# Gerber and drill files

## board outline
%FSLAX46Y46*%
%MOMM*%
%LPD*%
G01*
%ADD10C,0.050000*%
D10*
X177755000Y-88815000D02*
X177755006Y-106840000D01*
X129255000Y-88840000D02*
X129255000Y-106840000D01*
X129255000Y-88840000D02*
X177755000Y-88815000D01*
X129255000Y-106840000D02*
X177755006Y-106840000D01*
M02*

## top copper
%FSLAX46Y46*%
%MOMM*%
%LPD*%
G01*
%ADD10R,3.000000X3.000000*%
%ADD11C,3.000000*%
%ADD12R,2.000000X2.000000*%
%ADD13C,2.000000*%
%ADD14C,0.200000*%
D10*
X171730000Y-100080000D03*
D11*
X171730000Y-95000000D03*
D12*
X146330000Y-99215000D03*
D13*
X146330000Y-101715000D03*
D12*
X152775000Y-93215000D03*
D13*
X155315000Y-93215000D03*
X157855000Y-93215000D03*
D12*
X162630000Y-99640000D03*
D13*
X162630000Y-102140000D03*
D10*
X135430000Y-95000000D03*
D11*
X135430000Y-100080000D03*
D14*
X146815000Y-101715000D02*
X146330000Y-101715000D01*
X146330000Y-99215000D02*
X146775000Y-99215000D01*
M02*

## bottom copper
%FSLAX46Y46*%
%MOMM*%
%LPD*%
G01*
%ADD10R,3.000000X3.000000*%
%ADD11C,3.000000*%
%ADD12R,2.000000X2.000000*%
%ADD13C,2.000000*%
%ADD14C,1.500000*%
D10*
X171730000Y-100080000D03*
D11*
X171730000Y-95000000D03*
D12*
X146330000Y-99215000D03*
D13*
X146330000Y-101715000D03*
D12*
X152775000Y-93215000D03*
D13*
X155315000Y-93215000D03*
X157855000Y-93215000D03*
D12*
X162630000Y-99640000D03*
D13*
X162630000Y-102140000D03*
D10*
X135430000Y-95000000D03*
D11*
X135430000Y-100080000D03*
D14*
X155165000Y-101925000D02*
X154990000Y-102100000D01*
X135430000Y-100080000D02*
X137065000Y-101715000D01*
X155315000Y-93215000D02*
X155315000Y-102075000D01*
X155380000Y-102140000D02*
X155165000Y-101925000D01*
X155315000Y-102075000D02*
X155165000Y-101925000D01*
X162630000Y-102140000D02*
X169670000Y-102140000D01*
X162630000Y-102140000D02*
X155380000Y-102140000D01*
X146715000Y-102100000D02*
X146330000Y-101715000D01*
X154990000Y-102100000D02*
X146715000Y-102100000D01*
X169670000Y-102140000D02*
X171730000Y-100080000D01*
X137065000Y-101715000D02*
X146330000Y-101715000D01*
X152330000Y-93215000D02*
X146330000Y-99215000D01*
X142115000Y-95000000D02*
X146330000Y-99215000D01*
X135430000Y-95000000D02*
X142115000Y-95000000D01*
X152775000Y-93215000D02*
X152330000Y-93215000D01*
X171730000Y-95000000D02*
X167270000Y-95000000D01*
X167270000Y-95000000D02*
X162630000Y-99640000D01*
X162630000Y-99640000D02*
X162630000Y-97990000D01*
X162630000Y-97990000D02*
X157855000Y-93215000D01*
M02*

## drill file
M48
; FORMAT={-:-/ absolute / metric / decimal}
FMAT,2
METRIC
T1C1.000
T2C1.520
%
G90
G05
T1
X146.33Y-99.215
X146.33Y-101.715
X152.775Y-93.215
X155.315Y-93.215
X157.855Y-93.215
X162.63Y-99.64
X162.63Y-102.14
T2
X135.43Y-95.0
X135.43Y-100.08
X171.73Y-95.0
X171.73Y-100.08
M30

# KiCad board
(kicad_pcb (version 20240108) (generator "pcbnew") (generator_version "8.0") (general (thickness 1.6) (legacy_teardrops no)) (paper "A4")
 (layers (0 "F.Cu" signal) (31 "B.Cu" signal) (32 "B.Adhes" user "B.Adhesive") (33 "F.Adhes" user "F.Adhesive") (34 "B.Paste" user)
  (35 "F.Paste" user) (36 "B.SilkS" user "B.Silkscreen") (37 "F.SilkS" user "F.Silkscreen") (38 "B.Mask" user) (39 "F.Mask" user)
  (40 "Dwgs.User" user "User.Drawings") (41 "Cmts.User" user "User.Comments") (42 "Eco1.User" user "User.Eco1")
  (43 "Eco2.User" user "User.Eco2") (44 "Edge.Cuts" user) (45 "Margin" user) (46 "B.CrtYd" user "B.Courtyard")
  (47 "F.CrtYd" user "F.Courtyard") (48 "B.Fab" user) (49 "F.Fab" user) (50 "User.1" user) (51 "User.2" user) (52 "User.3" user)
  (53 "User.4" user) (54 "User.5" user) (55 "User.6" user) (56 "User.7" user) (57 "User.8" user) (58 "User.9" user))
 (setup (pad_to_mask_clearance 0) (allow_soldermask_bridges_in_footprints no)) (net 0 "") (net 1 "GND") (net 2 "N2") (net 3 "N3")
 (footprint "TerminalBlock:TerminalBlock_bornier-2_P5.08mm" (layer "F.Cu") (at 171.73 100.08 90)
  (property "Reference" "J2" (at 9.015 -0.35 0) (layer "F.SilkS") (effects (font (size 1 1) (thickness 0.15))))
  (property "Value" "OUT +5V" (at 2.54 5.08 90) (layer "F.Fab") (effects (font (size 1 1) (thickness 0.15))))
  (pad "1" thru_hole rect (at 0 0 90) (size 3 3) (drill 1.52) (layers "*.Cu" "*.Mask") (remove_unused_layers no) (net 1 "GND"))
  (pad "2" thru_hole circle (at 5.08 0 90) (size 3 3) (drill 1.52) (layers "*.Cu" "*.Mask") (remove_unused_layers no) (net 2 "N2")))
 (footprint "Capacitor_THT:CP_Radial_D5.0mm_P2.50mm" (layer "F.Cu") (at 146.33 99.215 -90)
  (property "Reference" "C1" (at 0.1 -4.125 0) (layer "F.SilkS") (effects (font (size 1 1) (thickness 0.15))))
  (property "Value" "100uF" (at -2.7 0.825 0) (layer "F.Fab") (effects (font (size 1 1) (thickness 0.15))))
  (pad "1" thru_hole rect (at 0 0 270) (size 2 2) (drill 1) (layers "*.Cu" "*.Mask") (remove_unused_layers no) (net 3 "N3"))
  (pad "2" thru_hole circle (at 2.5 0 270) (size 2 2) (drill 1) (layers "*.Cu" "*.Mask") (remove_unused_layers no) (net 1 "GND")))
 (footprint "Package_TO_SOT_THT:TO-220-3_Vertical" (layer "F.Cu") (at 152.775 93.215)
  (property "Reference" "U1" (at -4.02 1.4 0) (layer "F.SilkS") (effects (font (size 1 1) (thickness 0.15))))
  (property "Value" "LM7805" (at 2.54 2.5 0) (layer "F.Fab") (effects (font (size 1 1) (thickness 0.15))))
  (pad "1" thru_hole rect (at 0 0) (size 2 2) (drill 1) (layers "*.Cu" "*.Mask") (remove_unused_layers no) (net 3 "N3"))
  (pad "2" thru_hole circle (at 2.54 0) (size 2 2) (drill 1) (layers "*.Cu" "*.Mask") (remove_unused_layers no) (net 1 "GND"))
  (pad "3" thru_hole circle (at 5.08 0) (size 2 2) (drill 1) (layers "*.Cu" "*.Mask") (remove_unused_layers no) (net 2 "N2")))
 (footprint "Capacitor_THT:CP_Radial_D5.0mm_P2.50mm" (layer "F.Cu") (at 162.63 99.64 -90)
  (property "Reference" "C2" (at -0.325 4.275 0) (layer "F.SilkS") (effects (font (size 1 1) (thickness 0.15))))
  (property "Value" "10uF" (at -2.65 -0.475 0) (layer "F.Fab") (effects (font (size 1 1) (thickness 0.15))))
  (pad "1" thru_hole rect (at 0 0 270) (size 2 2) (drill 1) (layers "*.Cu" "*.Mask") (remove_unused_layers no) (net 2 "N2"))
  (pad "2" thru_hole circle (at 2.5 0 270) (size 2 2) (drill 1) (layers "*.Cu" "*.Mask") (remove_unused_layers no) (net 1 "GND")))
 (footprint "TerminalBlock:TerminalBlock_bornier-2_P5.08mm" (layer "F.Cu") (at 135.43 95 -90)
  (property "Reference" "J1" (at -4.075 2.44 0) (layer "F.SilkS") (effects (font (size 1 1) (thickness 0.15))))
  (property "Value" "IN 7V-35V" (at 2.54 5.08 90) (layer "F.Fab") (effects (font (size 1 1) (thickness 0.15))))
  (pad "1" thru_hole rect (at 0 0 270) (size 3 3) (drill 1.52) (layers "*.Cu" "*.Mask") (remove_unused_layers no) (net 3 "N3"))
  (pad "2" thru_hole circle (at 5.08 0 270) (size 3 3) (drill 1.52) (layers "*.Cu" "*.Mask") (remove_unused_layers no) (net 1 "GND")))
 (gr_line (start 177.755 88.815) (end 177.755006 106.84) (stroke (width 0.05) (type default)) (layer "Edge.Cuts"))
 (gr_line (start 129.255 88.84) (end 129.255 106.84) (stroke (width 0.05) (type default)) (layer "Edge.Cuts"))
 (gr_line (start 129.255 88.84) (end 177.755 88.815) (stroke (width 0.05) (type default)) (layer "Edge.Cuts"))
 (gr_line (start 129.255 106.84) (end 177.755006 106.84) (stroke (width 0.05) (type default)) (layer "Edge.Cuts"))
 (segment (start 146.815 101.715) (end 146.33 101.715) (width 0.2) (layer "F.Cu") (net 1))
 (segment (start 155.165 101.925) (end 154.99 102.1) (width 1.5) (layer "B.Cu") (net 1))
 (segment (start 135.43 100.08) (end 137.065 101.715) (width 1.5) (layer "B.Cu") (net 1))
 (segment (start 155.315 93.215) (end 155.315 102.075) (width 1.5) (layer "B.Cu") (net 1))
 (segment (start 155.38 102.14) (end 155.165 101.925) (width 1.5) (layer "B.Cu") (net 1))
 (segment (start 155.315 102.075) (end 155.165 101.925) (width 1.5) (layer "B.Cu") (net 1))
 (segment (start 162.63 102.14) (end 169.67 102.14) (width 1.5) (layer "B.Cu") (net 1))
 (segment (start 162.63 102.14) (end 155.38 102.14) (width 1.5) (layer "B.Cu") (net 1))
 (segment (start 146.715 102.1) (end 146.33 101.715) (width 1.5) (layer "B.Cu") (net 1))
 (segment (start 154.99 102.1) (end 146.715 102.1) (width 1.5) (layer "B.Cu") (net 1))
 (segment (start 169.67 102.14) (end 171.73 100.08) (width 1.5) (layer "B.Cu") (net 1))
 (segment (start 137.065 101.715) (end 146.33 101.715) (width 1.5) (layer "B.Cu") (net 1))
 (segment (start 146.33 99.215) (end 146.775 99.215) (width 0.2) (layer "F.Cu") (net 3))
 (segment (start 152.33 93.215) (end 146.33 99.215) (width 1.5) (layer "B.Cu") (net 3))
 (segment (start 142.115 95) (end 146.33 99.215) (width 1.5) (layer "B.Cu") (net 3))
 (segment (start 135.43 95) (end 142.115 95) (width 1.5) (layer "B.Cu") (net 3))
 (segment (start 152.775 93.215) (end 152.33 93.215) (width 1.5) (layer "B.Cu") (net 3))
 (segment (start 171.73 95) (end 167.27 95) (width 1.5) (layer "B.Cu") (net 2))
 (segment (start 167.27 95) (end 162.63 99.64) (width 1.5) (layer "B.Cu") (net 2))
 (segment (start 162.63 99.64) (end 162.63 97.99) (width 1.5) (layer "B.Cu") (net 2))
 (segment (start 162.63 97.99) (end 157.855 93.215) (width 1.5) (layer "B.Cu") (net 2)))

